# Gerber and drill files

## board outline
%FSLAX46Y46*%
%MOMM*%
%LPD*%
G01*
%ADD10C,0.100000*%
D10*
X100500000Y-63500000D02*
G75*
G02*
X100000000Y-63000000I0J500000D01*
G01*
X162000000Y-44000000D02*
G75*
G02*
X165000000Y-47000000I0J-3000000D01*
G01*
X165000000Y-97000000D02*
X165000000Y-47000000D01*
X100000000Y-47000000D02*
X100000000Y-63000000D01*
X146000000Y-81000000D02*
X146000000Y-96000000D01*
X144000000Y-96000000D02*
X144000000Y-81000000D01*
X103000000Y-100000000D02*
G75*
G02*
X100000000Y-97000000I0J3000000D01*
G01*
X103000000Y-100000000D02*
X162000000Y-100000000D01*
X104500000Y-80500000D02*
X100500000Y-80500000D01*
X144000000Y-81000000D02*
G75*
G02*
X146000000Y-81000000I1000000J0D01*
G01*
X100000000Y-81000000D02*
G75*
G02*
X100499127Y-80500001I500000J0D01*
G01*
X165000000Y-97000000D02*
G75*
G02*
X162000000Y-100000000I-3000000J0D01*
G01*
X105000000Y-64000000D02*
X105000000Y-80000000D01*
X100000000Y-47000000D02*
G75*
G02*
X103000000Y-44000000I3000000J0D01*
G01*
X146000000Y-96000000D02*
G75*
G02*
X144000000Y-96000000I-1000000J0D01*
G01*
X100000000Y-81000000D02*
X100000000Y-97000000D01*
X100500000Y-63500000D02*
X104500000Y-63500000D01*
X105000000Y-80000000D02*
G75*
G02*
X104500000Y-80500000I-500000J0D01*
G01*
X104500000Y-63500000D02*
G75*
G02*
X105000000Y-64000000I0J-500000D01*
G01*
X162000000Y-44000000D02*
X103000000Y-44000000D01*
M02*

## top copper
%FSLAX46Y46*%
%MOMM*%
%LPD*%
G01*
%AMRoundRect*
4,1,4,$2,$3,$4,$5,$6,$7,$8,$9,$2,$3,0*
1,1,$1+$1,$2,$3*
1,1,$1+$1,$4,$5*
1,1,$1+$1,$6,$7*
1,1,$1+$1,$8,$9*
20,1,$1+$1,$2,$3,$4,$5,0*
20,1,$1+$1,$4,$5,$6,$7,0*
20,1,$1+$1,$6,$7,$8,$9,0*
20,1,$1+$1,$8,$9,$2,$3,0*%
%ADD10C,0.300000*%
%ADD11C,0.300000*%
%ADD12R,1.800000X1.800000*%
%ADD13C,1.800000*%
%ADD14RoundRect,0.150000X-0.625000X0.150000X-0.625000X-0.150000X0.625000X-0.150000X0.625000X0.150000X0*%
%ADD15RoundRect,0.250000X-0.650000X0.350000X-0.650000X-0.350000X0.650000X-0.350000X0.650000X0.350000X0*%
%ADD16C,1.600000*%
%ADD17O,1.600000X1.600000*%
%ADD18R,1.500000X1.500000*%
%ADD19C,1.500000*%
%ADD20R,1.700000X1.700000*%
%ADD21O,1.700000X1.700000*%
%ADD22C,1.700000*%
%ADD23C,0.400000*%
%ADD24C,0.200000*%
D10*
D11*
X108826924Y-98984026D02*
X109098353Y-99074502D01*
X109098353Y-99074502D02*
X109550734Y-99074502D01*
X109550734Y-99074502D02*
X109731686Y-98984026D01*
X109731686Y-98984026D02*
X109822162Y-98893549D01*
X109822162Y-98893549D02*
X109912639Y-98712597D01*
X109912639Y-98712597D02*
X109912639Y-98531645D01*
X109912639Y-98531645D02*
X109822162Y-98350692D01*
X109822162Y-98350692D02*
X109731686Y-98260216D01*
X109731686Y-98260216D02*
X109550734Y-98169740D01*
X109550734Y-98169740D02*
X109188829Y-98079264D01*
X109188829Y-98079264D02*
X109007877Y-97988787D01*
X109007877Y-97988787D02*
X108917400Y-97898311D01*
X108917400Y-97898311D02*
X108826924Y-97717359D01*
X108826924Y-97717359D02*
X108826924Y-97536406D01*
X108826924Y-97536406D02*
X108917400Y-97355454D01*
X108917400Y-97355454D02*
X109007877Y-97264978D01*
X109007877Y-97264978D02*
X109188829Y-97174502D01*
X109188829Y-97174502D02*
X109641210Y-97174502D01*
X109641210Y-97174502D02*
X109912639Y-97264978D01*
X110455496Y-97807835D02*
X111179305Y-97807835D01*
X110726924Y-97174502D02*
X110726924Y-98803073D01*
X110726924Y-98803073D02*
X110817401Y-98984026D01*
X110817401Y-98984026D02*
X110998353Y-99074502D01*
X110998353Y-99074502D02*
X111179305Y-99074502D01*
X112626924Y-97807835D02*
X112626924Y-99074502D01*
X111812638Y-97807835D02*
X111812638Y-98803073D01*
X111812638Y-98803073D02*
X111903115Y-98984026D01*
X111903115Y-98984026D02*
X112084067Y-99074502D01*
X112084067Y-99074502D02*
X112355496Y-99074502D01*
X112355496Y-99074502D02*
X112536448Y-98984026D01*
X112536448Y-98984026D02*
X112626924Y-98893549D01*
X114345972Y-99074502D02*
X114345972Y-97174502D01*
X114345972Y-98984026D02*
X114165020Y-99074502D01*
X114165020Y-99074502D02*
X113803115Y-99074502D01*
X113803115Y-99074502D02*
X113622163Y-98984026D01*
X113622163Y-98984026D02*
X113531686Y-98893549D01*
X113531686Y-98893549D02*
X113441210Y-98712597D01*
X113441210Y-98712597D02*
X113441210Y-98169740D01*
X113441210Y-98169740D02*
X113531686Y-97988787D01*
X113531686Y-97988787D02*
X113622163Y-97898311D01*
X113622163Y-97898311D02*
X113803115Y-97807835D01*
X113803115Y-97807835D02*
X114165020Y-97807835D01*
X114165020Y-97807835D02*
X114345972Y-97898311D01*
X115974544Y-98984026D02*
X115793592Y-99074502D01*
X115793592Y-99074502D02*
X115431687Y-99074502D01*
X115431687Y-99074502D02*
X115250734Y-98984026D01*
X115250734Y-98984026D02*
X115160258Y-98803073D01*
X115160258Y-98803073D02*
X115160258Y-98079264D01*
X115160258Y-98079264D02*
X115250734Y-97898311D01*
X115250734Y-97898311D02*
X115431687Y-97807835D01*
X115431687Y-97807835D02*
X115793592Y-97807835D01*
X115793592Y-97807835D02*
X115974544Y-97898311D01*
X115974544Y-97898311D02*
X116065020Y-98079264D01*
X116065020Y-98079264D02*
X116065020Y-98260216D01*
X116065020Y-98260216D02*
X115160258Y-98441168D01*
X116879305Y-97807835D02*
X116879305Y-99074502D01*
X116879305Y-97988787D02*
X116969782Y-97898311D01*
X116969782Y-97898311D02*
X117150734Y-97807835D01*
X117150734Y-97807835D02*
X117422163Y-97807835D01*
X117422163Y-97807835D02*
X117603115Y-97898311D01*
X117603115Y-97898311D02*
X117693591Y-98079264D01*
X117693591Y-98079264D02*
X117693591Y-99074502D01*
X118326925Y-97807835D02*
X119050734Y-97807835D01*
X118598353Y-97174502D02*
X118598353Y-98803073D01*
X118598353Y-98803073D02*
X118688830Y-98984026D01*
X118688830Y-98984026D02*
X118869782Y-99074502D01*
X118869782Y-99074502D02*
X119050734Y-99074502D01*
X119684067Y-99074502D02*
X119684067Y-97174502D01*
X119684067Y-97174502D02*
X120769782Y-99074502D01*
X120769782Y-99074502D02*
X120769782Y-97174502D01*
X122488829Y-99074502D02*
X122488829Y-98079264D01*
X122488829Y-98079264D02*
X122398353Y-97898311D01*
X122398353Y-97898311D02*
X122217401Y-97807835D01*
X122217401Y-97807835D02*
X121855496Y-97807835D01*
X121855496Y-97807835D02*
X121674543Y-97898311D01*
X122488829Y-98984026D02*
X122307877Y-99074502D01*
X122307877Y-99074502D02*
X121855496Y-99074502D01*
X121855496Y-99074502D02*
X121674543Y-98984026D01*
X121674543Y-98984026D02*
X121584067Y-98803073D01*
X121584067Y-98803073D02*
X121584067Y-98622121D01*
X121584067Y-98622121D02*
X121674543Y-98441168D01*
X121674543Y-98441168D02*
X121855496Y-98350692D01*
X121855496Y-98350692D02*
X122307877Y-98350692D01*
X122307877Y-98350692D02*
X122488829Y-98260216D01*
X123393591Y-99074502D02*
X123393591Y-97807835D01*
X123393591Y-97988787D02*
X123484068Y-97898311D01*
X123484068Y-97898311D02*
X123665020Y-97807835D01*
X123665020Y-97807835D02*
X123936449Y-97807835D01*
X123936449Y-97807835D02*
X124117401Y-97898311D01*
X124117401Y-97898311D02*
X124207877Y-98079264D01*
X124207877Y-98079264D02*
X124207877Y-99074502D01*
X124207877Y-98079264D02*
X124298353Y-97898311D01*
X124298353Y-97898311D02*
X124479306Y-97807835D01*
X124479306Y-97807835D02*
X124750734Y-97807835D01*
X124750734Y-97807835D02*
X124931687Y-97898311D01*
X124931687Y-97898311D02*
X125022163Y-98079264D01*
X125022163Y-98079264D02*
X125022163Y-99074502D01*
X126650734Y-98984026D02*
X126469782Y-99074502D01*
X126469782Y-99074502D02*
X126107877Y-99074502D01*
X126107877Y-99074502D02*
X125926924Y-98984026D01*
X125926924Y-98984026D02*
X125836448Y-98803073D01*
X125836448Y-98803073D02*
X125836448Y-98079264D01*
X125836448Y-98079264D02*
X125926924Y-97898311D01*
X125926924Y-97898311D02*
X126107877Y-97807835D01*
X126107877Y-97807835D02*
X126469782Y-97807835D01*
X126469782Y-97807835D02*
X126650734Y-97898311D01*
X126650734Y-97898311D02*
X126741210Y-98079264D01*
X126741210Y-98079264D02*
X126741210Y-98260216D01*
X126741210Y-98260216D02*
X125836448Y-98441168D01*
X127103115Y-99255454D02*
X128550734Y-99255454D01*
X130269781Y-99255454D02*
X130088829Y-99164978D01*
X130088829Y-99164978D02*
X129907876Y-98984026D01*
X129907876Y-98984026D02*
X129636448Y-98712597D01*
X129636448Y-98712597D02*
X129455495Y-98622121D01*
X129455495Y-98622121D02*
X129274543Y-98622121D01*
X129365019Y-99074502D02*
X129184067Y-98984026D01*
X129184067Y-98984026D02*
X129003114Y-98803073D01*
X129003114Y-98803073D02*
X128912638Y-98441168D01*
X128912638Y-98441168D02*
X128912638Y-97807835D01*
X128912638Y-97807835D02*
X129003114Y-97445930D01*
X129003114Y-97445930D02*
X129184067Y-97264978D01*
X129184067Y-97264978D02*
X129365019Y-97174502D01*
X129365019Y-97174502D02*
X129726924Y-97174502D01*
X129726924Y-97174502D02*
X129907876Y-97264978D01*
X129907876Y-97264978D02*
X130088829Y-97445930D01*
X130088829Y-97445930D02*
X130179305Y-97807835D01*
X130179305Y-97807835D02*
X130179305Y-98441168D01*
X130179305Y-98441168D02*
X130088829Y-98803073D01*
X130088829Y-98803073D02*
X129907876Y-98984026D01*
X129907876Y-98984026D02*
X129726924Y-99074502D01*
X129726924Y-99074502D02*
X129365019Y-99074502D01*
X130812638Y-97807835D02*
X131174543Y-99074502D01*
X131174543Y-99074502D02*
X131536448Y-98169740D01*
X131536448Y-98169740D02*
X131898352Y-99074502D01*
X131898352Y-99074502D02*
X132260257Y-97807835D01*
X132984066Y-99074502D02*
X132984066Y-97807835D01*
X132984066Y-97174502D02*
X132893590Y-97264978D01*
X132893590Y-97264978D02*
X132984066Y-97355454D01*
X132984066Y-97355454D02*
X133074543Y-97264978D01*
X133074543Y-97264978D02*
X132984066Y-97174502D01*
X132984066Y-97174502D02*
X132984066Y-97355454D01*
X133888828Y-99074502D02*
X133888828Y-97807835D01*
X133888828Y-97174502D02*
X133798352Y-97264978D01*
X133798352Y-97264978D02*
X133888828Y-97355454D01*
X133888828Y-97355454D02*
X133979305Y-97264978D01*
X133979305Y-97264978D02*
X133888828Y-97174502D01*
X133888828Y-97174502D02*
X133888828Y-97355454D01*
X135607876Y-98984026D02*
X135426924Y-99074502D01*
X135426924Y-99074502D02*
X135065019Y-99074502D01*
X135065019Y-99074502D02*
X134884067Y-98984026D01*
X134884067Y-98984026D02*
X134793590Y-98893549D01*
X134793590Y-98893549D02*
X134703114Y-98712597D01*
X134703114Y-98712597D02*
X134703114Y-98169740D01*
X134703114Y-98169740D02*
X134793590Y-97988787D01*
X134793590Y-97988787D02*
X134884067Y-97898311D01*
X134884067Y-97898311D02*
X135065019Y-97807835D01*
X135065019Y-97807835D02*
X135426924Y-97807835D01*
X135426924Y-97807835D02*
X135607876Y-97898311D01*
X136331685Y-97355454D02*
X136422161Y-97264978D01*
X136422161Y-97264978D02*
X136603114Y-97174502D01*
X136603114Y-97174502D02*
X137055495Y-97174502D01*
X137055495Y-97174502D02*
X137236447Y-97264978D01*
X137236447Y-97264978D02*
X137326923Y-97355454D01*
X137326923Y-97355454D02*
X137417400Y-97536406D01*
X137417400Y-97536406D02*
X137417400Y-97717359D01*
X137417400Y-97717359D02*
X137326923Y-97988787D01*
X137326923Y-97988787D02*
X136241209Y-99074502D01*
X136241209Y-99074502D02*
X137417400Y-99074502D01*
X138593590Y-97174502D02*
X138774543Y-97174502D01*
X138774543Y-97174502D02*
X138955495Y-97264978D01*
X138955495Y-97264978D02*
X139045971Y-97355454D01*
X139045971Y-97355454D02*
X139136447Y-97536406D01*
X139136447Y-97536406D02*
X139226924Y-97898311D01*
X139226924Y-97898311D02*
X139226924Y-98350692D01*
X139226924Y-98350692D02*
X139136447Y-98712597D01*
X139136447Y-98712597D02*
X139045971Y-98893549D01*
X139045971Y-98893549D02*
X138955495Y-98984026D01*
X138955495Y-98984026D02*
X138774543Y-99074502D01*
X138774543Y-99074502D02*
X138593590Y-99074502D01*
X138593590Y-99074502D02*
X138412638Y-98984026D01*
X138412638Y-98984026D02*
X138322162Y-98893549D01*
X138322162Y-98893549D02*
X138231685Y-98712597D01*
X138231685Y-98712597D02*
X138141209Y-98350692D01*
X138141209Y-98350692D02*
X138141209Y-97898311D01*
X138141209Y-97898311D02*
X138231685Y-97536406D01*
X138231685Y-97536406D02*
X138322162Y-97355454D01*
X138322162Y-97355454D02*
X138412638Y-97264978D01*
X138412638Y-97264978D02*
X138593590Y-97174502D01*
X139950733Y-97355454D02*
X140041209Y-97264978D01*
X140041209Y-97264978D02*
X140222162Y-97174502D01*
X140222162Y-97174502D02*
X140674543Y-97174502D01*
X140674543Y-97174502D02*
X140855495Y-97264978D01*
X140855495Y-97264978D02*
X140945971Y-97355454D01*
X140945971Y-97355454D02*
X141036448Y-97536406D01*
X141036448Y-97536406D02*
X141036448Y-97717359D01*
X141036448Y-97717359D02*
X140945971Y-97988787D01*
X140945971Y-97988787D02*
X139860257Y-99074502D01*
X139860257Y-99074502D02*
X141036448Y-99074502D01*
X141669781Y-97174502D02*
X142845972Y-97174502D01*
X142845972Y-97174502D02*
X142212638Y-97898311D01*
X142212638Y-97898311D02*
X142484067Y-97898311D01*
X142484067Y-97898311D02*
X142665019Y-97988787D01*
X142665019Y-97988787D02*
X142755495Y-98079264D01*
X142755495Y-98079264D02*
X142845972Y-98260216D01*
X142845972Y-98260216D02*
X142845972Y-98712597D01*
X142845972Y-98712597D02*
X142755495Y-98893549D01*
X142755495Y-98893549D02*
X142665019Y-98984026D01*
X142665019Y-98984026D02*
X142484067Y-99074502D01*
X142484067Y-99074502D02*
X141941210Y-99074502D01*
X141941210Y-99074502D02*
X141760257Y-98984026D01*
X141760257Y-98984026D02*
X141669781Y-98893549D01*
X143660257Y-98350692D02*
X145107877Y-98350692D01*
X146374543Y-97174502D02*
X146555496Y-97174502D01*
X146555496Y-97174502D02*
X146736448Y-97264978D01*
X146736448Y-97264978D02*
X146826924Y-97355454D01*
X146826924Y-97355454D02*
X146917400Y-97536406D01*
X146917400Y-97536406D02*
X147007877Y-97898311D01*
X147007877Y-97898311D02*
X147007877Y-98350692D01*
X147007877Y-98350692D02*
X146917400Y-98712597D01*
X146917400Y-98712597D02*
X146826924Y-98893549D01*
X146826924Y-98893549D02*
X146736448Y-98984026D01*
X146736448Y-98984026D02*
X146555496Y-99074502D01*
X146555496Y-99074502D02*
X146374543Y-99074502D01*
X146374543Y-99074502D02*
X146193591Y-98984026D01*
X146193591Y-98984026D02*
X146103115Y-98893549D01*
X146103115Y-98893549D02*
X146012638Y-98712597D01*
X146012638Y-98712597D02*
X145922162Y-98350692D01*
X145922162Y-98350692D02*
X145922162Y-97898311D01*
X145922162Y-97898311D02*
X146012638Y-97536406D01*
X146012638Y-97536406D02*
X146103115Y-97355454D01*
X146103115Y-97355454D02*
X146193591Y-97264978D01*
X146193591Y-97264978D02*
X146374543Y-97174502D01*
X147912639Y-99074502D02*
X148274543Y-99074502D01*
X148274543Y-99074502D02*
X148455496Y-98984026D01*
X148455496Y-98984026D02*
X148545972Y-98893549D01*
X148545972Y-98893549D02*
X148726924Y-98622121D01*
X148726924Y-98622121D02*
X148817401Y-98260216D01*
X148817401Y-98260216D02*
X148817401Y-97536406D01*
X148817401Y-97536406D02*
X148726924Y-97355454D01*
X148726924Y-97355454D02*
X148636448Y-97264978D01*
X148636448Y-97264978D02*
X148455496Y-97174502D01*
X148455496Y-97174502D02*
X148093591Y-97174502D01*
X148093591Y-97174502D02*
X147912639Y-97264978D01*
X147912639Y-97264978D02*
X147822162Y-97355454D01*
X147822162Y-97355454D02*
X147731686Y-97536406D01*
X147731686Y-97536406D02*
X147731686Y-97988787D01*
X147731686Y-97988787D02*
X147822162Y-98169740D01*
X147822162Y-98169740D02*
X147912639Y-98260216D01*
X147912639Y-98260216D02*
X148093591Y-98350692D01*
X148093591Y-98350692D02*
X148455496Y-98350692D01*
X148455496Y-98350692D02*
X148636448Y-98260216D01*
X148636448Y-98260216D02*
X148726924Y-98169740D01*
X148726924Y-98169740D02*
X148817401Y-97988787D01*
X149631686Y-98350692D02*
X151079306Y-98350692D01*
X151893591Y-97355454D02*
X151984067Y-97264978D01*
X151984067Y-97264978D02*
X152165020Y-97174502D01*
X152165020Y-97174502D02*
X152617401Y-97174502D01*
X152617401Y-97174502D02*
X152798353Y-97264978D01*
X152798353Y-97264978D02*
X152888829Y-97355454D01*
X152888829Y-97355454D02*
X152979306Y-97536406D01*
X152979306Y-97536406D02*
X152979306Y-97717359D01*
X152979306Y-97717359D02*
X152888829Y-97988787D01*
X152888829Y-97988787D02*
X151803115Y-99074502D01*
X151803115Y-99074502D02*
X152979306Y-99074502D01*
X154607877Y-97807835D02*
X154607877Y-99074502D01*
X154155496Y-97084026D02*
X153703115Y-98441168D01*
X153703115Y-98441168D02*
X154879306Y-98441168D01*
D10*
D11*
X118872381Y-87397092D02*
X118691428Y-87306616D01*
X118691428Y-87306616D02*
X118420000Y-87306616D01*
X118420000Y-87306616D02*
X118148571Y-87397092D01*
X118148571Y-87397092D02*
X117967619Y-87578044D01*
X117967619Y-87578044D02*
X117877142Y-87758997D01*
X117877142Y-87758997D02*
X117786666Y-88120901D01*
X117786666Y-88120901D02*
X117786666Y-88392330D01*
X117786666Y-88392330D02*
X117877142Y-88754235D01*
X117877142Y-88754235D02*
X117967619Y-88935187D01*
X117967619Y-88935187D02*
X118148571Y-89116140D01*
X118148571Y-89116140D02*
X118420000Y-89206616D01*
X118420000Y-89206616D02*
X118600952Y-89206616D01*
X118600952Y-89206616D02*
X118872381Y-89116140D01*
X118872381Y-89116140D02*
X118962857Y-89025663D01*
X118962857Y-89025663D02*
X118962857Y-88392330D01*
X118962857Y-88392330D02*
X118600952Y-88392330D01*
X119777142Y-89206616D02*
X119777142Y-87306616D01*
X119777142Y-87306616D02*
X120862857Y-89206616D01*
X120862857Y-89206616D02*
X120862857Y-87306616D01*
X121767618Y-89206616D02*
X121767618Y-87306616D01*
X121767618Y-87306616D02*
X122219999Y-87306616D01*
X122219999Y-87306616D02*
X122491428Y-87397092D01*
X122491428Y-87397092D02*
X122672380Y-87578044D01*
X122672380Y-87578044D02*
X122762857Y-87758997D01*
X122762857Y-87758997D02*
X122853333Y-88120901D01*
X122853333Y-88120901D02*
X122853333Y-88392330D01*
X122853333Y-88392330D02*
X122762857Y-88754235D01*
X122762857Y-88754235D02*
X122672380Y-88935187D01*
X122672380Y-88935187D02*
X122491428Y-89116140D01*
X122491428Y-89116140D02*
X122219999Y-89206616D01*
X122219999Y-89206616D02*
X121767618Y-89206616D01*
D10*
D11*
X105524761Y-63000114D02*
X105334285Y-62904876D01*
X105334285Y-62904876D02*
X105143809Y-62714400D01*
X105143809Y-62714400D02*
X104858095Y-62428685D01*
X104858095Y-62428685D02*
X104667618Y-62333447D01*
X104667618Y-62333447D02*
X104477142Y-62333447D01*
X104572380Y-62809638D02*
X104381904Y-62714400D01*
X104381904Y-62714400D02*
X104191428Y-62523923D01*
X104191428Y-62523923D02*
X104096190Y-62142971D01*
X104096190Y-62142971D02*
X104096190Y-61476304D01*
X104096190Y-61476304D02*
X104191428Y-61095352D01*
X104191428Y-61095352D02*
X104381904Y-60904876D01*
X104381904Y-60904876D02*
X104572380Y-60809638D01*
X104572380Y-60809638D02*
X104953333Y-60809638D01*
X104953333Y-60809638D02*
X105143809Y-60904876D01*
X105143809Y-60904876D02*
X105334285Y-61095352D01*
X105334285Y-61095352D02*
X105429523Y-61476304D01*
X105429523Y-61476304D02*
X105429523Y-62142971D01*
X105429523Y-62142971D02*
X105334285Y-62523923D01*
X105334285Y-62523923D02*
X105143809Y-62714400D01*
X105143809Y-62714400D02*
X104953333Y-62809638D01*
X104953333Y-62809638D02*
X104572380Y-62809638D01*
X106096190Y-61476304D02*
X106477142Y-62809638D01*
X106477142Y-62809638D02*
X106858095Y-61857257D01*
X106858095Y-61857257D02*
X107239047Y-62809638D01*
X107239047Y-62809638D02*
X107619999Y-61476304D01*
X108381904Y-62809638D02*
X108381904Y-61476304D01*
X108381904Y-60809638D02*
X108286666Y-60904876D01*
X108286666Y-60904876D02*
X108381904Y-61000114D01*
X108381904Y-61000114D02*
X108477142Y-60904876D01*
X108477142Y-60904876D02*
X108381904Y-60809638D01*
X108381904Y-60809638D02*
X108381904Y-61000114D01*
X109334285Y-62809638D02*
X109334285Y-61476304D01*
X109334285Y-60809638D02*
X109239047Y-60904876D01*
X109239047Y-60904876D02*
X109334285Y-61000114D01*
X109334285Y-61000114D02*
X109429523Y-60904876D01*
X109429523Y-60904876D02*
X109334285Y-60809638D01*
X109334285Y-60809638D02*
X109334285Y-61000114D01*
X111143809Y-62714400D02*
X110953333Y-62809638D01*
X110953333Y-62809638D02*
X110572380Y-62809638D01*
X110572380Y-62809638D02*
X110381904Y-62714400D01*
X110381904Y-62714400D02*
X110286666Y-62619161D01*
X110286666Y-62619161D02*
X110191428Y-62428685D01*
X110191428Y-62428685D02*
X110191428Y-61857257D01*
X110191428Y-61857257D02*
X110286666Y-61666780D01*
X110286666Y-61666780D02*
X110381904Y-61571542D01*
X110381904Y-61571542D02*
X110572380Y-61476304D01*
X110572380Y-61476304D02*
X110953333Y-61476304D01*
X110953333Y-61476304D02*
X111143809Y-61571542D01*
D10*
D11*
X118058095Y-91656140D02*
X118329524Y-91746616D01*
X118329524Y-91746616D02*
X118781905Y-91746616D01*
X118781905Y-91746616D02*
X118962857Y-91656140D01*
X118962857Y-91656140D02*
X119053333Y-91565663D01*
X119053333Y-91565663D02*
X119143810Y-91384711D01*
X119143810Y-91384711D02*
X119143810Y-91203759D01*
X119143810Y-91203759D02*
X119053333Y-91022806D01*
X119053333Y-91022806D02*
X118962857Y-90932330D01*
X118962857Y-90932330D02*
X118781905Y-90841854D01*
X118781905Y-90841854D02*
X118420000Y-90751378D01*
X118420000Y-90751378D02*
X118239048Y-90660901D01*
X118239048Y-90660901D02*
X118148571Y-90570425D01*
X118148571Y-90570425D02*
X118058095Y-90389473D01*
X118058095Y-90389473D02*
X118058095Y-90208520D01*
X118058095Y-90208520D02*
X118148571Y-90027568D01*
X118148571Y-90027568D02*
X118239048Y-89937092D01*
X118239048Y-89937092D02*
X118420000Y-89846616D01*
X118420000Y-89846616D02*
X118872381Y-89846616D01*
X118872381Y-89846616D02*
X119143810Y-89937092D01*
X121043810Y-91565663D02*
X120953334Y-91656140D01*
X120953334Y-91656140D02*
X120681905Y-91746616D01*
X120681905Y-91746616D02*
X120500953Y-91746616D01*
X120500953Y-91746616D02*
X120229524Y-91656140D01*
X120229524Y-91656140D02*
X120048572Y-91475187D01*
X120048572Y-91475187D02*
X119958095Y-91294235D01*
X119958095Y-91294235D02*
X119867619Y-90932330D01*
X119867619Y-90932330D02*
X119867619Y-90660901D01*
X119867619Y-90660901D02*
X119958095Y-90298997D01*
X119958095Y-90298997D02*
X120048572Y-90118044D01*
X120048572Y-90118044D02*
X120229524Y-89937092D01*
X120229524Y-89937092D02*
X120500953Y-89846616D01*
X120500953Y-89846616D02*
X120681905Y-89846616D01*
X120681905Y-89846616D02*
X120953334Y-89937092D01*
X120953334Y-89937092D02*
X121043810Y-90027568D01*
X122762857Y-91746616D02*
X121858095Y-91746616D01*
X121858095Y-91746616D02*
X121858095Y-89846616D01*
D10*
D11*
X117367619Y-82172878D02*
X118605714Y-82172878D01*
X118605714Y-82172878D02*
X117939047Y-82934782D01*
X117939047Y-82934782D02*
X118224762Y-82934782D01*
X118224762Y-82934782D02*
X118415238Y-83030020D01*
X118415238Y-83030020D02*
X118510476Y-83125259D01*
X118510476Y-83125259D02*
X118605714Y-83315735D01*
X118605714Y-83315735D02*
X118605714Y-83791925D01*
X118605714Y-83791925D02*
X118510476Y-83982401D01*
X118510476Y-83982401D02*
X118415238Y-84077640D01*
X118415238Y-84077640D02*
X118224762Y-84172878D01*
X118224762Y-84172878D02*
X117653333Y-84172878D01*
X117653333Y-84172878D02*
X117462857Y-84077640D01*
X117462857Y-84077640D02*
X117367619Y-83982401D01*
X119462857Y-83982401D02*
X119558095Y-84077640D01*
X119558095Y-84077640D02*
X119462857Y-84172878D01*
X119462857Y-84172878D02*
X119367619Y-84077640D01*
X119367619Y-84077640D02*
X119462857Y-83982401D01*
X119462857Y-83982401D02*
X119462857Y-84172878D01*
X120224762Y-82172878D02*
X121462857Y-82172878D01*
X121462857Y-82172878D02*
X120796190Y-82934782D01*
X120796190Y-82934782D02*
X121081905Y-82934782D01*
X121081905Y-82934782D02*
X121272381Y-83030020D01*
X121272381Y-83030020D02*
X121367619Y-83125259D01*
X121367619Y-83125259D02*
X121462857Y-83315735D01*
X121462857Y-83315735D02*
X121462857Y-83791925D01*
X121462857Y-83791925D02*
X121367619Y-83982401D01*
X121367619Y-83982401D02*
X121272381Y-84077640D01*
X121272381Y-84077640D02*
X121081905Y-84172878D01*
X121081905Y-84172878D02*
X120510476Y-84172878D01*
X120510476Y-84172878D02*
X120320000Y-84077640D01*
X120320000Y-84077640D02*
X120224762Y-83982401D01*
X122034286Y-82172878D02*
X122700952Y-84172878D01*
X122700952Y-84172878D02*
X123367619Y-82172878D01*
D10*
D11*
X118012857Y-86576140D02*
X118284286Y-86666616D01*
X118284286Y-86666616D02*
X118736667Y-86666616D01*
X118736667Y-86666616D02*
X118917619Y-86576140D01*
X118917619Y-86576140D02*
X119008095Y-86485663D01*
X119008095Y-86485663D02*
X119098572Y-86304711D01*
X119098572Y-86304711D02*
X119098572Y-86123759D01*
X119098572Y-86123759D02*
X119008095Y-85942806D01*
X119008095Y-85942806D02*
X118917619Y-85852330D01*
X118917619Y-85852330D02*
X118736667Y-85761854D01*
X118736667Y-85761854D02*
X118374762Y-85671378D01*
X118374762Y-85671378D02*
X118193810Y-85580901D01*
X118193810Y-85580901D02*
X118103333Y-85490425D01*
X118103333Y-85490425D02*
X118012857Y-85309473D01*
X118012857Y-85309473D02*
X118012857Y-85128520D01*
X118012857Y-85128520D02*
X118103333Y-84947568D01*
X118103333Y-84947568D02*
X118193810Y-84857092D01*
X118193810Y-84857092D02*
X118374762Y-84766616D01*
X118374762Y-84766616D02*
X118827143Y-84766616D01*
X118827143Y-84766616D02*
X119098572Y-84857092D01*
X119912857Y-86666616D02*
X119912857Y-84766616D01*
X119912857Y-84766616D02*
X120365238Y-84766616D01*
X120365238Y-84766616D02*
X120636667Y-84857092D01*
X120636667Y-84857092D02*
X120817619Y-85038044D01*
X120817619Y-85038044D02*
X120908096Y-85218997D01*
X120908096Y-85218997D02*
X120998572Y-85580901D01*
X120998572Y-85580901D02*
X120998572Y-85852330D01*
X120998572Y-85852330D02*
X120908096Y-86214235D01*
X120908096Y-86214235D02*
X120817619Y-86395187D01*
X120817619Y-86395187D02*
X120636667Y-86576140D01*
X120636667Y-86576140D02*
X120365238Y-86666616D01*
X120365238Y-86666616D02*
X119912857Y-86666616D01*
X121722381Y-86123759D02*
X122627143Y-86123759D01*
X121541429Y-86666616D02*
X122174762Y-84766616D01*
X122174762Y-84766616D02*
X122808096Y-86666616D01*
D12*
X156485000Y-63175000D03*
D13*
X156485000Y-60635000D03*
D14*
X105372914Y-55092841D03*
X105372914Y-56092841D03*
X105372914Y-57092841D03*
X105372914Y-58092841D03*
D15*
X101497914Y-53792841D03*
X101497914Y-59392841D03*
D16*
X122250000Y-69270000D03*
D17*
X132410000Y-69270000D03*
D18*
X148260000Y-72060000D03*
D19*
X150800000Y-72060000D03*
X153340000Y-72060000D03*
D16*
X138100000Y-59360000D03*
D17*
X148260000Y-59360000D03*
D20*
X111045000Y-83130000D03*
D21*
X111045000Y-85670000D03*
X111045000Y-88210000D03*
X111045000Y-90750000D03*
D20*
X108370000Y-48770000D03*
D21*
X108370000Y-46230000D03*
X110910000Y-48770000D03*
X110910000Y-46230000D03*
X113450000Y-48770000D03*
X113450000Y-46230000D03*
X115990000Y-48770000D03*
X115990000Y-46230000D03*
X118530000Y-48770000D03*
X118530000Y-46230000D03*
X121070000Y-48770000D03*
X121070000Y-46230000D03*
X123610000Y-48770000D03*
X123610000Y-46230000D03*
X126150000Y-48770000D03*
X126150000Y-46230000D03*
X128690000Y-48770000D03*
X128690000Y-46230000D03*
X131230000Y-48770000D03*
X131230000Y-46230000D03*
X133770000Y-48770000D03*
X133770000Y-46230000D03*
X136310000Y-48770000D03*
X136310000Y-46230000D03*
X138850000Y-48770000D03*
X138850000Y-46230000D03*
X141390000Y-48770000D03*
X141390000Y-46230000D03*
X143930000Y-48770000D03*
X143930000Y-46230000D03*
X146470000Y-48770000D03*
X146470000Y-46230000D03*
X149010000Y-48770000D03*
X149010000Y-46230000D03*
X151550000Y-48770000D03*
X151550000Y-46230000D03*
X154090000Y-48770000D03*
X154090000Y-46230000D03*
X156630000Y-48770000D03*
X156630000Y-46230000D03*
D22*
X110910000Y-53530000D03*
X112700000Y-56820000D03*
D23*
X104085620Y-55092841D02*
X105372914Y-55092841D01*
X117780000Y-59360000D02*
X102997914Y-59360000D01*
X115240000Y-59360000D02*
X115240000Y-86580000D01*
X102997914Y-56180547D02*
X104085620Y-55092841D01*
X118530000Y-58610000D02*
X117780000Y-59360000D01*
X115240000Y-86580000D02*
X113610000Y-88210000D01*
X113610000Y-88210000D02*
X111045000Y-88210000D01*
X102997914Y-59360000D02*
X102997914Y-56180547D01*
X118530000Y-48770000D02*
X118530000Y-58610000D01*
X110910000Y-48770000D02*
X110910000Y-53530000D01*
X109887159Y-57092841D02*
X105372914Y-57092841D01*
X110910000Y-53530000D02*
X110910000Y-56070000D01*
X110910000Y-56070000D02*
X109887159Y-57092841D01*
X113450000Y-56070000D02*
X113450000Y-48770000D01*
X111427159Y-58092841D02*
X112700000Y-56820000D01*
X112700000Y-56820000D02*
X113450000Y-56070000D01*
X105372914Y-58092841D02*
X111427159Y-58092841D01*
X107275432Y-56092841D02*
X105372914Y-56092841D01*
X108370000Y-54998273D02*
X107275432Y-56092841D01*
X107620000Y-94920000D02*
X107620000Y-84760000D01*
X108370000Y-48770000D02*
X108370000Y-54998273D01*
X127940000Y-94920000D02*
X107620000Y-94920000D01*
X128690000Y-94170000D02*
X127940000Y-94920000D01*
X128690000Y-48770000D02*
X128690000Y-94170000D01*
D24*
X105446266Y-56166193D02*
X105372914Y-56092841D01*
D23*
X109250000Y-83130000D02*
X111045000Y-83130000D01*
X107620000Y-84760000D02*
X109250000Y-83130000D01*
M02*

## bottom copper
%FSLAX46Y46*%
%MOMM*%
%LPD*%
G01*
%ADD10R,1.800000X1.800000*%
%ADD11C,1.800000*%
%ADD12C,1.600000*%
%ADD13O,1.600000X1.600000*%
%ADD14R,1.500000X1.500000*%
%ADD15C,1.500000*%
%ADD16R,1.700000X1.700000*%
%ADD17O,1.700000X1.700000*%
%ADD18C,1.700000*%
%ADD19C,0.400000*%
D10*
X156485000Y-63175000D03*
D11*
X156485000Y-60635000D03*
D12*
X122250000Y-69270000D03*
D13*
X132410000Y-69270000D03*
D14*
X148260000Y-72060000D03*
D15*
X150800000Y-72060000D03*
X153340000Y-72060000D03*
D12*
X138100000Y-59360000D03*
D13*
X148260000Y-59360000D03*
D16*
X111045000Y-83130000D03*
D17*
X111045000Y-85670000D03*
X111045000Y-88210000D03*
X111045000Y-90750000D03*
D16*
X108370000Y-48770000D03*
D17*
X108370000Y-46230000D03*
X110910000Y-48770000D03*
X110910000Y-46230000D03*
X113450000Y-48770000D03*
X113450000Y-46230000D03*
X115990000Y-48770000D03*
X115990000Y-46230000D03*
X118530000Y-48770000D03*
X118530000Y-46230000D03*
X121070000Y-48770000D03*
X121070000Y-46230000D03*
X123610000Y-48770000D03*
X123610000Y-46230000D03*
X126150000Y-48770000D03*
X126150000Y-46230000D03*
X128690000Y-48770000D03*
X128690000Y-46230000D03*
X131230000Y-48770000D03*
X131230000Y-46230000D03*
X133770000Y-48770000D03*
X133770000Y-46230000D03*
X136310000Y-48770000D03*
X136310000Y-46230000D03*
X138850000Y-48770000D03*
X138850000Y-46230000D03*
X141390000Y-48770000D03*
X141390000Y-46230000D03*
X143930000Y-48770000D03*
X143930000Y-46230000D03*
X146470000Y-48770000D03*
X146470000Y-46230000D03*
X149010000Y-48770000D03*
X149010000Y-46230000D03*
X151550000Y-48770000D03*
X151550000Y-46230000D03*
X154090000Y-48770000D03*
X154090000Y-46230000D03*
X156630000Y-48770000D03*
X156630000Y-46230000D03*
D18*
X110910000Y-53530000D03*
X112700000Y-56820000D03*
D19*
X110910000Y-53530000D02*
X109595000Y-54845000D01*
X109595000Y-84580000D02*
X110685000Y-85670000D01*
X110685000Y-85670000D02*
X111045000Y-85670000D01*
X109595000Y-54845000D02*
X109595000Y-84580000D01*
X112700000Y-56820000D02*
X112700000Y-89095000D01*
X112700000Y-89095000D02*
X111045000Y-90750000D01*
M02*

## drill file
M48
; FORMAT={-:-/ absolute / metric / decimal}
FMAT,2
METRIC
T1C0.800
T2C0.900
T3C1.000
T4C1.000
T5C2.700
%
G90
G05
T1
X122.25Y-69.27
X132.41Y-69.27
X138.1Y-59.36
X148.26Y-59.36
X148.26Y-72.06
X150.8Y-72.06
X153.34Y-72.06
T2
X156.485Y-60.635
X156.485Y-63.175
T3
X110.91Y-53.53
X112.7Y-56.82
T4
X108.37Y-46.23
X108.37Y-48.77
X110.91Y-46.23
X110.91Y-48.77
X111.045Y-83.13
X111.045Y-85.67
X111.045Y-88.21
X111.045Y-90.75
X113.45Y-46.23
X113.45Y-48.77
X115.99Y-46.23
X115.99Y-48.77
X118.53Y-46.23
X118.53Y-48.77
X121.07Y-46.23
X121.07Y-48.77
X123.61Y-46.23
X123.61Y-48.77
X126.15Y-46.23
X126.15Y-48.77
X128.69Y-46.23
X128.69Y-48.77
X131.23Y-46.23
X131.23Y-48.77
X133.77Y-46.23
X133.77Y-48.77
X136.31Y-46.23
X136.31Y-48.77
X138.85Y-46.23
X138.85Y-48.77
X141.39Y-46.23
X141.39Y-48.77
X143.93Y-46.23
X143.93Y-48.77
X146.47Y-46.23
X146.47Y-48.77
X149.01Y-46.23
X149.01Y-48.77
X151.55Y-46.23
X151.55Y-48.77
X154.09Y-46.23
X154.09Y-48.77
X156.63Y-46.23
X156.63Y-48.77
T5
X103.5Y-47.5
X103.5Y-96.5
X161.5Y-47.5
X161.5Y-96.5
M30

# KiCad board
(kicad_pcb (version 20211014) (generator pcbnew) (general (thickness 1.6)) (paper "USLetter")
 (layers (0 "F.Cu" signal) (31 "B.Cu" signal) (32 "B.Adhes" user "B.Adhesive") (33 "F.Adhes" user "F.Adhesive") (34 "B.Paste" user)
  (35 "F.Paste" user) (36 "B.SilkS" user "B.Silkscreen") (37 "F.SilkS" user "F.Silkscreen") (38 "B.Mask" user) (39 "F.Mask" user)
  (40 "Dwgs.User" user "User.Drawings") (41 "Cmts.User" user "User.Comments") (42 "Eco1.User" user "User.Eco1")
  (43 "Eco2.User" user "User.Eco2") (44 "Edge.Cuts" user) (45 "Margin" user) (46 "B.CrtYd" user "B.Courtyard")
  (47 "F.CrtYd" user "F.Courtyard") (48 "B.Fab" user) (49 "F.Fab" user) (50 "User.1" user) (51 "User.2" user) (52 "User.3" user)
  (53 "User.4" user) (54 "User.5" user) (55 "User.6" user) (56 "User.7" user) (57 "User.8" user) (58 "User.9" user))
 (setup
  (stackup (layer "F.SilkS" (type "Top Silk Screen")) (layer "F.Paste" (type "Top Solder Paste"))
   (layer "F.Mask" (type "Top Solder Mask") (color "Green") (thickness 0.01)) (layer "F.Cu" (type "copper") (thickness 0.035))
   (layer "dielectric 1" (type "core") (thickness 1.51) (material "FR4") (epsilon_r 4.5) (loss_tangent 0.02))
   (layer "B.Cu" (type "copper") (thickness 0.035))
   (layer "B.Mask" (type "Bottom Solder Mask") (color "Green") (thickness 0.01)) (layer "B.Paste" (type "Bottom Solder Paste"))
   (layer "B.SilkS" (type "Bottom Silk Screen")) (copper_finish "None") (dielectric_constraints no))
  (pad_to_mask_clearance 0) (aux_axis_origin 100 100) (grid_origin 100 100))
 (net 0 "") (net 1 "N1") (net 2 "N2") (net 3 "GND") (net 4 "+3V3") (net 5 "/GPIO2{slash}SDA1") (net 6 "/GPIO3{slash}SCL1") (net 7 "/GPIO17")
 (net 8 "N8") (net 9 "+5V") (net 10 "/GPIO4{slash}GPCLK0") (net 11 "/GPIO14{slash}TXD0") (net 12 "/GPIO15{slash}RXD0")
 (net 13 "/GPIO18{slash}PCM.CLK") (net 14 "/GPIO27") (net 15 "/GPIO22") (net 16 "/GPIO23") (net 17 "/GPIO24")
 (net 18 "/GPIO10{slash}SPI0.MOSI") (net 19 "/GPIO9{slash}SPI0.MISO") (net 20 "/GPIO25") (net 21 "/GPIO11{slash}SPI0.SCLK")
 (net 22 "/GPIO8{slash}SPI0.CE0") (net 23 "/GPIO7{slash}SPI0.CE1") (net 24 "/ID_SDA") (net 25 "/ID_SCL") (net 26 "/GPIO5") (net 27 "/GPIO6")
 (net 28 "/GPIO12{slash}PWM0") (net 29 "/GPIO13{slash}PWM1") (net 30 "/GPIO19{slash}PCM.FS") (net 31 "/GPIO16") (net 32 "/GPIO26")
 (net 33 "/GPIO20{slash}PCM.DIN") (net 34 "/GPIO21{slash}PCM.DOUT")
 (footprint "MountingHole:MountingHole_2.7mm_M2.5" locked (layer "F.Cu") (at 161.5 47.5)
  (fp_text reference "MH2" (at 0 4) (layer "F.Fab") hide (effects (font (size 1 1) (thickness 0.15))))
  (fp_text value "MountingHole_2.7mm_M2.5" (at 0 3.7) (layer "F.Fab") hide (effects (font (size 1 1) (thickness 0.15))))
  (pad "" np_thru_hole circle locked (at 0 0) (size 2.7 2.7) (drill 2.7) (layers *.Cu *.Mask)))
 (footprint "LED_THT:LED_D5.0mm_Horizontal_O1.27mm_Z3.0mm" (layer "F.Cu") (at 156.485 63.175 90)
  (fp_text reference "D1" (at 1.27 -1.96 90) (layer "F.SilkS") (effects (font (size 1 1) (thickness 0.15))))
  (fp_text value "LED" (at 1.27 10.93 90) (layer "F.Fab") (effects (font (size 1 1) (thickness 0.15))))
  (pad "1" thru_hole rect (at 0 0 90) (size 1.8 1.8) (drill 0.9) (layers *.Cu *.Mask) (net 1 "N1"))
  (pad "2" thru_hole circle (at 2.54 0 90) (size 1.8 1.8) (drill 0.9) (layers *.Cu *.Mask) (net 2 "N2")))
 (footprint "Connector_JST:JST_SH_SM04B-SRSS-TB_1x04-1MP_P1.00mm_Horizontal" (layer "F.Cu") (at 103.372914 56.592841 -90)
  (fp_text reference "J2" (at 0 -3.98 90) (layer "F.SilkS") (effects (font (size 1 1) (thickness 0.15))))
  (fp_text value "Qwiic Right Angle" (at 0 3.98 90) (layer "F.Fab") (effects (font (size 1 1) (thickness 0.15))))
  (pad "1" smd roundrect (at -1.5 -2 270) (size 0.6 1.55) (layers "F.Cu" "F.Paste" "F.Mask") (roundrect_rratio 0.25) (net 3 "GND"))
  (pad "2" smd roundrect (at -0.5 -2 270) (size 0.6 1.55) (layers "F.Cu" "F.Paste" "F.Mask") (roundrect_rratio 0.25) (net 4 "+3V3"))
  (pad "3" smd roundrect (at 0.5 -2 270) (size 0.6 1.55) (layers "F.Cu" "F.Paste" "F.Mask") (roundrect_rratio 0.25)
   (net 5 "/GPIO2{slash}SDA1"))
  (pad "4" smd roundrect (at 1.5 -2 270) (size 0.6 1.55) (layers "F.Cu" "F.Paste" "F.Mask") (roundrect_rratio 0.25)
   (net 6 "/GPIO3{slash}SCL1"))
  (pad "MP" smd roundrect (at -2.8 1.875 270) (size 1.2 1.8) (layers "F.Cu" "F.Paste" "F.Mask") (roundrect_rratio 0.2083333333))
  (pad "MP" smd roundrect (at 2.8 1.875 270) (size 1.2 1.8) (layers "F.Cu" "F.Paste" "F.Mask") (roundrect_rratio 0.2083333333)))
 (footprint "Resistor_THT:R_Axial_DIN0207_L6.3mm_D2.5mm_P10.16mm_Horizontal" (layer "F.Cu") (at 122.25 69.27)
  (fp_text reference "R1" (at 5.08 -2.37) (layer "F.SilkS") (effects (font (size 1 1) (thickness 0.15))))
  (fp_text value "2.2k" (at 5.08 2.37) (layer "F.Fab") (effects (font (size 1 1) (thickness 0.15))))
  (pad "1" thru_hole circle (at 0 0) (size 1.6 1.6) (drill 0.8) (layers *.Cu *.Mask) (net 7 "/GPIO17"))
  (pad "2" thru_hole oval (at 10.16 0) (size 1.6 1.6) (drill 0.8) (layers *.Cu *.Mask) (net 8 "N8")))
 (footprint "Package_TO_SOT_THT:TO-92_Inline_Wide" (layer "F.Cu") (at 148.26 72.06)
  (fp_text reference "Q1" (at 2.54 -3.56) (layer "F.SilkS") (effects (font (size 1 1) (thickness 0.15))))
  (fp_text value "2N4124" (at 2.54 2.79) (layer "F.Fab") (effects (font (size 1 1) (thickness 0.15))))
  (pad "1" thru_hole rect (at 0 0) (size 1.5 1.5) (drill 0.8) (layers *.Cu *.Mask) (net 3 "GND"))
  (pad "2" thru_hole circle (at 2.54 0) (size 1.5 1.5) (drill 0.8) (layers *.Cu *.Mask) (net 8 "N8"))
  (pad "3" thru_hole circle (at 5.08 0) (size 1.5 1.5) (drill 0.8) (layers *.Cu *.Mask) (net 1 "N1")))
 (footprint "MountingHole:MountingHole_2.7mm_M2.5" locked (layer "F.Cu") (at 103.5 96.5)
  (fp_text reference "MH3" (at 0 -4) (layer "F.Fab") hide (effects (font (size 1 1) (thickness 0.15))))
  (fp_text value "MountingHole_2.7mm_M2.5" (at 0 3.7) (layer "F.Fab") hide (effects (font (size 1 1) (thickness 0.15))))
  (pad "" np_thru_hole circle locked (at 0 0) (size 2.7 2.7) (drill 2.7) (layers *.Cu *.Mask)))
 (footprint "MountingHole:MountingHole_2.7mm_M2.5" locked (layer "F.Cu") (at 103.5 47.5)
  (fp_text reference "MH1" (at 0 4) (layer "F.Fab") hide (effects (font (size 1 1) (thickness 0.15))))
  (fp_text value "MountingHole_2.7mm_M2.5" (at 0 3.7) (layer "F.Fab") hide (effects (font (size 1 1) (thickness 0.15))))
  (pad "" np_thru_hole circle locked (at 0 0) (size 2.7 2.7) (drill 2.7) (layers *.Cu *.Mask)))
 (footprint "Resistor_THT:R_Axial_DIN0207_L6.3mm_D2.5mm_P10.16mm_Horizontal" (layer "F.Cu") (at 138.1 59.36)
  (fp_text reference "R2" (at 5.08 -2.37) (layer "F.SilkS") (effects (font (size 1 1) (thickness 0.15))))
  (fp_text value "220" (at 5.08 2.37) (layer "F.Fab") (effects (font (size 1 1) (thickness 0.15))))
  (pad "1" thru_hole circle (at 0 0) (size 1.6 1.6) (drill 0.8) (layers *.Cu *.Mask) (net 4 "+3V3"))
  (pad "2" thru_hole oval (at 10.16 0) (size 1.6 1.6) (drill 0.8) (layers *.Cu *.Mask) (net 2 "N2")))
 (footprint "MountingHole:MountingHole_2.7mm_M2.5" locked (layer "F.Cu") (at 161.5 96.5)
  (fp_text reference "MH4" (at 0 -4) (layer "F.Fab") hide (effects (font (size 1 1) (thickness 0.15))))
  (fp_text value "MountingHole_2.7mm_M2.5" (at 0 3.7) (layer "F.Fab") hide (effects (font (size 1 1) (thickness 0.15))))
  (pad "" np_thru_hole circle locked (at 0 0) (size 2.7 2.7) (drill 2.7) (layers *.Cu *.Mask)))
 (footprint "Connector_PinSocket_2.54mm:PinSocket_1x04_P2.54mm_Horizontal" (layer "F.Cu") (at 111.045 83.13)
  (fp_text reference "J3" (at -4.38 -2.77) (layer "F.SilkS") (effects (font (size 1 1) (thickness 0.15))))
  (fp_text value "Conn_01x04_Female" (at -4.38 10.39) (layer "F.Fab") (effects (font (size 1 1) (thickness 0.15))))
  (pad "1" thru_hole rect (at 0 0) (size 1.7 1.7) (drill 1) (layers *.Cu *.Mask) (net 4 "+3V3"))
  (pad "2" thru_hole oval (at 0 2.54) (size 1.7 1.7) (drill 1) (layers *.Cu *.Mask) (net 5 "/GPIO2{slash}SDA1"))
  (pad "3" thru_hole oval (at 0 5.08) (size 1.7 1.7) (drill 1) (layers *.Cu *.Mask) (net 3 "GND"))
  (pad "4" thru_hole oval (at 0 7.62) (size 1.7 1.7) (drill 1) (layers *.Cu *.Mask) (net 6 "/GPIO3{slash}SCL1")))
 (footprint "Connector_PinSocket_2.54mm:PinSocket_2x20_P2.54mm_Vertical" (layer "B.Cu") (at 108.37 48.77 -90)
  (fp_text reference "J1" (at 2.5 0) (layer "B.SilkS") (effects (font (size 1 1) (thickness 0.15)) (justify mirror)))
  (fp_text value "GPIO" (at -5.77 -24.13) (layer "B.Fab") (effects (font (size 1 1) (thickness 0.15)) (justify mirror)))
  (pad "1" thru_hole rect locked (at 0 0 270) (size 1.7 1.7) (drill 1) (layers *.Cu *.Mask) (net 4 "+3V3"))
  (pad "2" thru_hole oval locked (at -2.54 0 270) (size 1.7 1.7) (drill 1) (layers *.Cu *.Mask) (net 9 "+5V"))
  (pad "3" thru_hole oval locked (at 0 -2.54 270) (size 1.7 1.7) (drill 1) (layers *.Cu *.Mask) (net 5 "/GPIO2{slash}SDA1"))
  (pad "4" thru_hole oval locked (at -2.54 -2.54 270) (size 1.7 1.7) (drill 1) (layers *.Cu *.Mask) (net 9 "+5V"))
  (pad "5" thru_hole oval locked (at 0 -5.08 270) (size 1.7 1.7) (drill 1) (layers *.Cu *.Mask) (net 6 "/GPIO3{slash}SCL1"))
  (pad "6" thru_hole oval locked (at -2.54 -5.08 270) (size 1.7 1.7) (drill 1) (layers *.Cu *.Mask) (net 3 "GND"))
  (pad "7" thru_hole oval locked (at 0 -7.62 270) (size 1.7 1.7) (drill 1) (layers *.Cu *.Mask) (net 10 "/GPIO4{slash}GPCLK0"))
  (pad "8" thru_hole oval locked (at -2.54 -7.62 270) (size 1.7 1.7) (drill 1) (layers *.Cu *.Mask) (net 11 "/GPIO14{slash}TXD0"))
  (pad "9" thru_hole oval locked (at 0 -10.16 270) (size 1.7 1.7) (drill 1) (layers *.Cu *.Mask) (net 3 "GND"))
  (pad "10" thru_hole oval locked (at -2.54 -10.16 270) (size 1.7 1.7) (drill 1) (layers *.Cu *.Mask) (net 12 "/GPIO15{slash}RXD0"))
  (pad "11" thru_hole oval locked (at 0 -12.7 270) (size 1.7 1.7) (drill 1) (layers *.Cu *.Mask) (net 7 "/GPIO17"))
  (pad "12" thru_hole oval locked (at -2.54 -12.7 270) (size 1.7 1.7) (drill 1) (layers *.Cu *.Mask) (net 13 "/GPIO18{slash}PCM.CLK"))
  (pad "13" thru_hole oval locked (at 0 -15.24 270) (size 1.7 1.7) (drill 1) (layers *.Cu *.Mask) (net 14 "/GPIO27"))
  (pad "14" thru_hole oval locked (at -2.54 -15.24 270) (size 1.7 1.7) (drill 1) (layers *.Cu *.Mask) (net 3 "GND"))
  (pad "15" thru_hole oval locked (at 0 -17.78 270) (size 1.7 1.7) (drill 1) (layers *.Cu *.Mask) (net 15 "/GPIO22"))
  (pad "16" thru_hole oval locked (at -2.54 -17.78 270) (size 1.7 1.7) (drill 1) (layers *.Cu *.Mask) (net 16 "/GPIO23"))
  (pad "17" thru_hole oval locked (at 0 -20.32 270) (size 1.7 1.7) (drill 1) (layers *.Cu *.Mask) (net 4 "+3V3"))
  (pad "18" thru_hole oval locked (at -2.54 -20.32 270) (size 1.7 1.7) (drill 1) (layers *.Cu *.Mask) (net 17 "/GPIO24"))
  (pad "19" thru_hole oval locked (at 0 -22.86 270) (size 1.7 1.7) (drill 1) (layers *.Cu *.Mask) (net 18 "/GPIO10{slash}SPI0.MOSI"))
  (pad "20" thru_hole oval locked (at -2.54 -22.86 270) (size 1.7 1.7) (drill 1) (layers *.Cu *.Mask) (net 3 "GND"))
  (pad "21" thru_hole oval locked (at 0 -25.4 270) (size 1.7 1.7) (drill 1) (layers *.Cu *.Mask) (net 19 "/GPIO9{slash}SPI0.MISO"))
  (pad "22" thru_hole oval locked (at -2.54 -25.4 270) (size 1.7 1.7) (drill 1) (layers *.Cu *.Mask) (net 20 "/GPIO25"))
  (pad "23" thru_hole oval locked (at 0 -27.94 270) (size 1.7 1.7) (drill 1) (layers *.Cu *.Mask) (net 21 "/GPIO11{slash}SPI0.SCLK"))
  (pad "24" thru_hole oval locked (at -2.54 -27.94 270) (size 1.7 1.7) (drill 1) (layers *.Cu *.Mask) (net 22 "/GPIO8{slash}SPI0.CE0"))
  (pad "25" thru_hole oval locked (at 0 -30.48 270) (size 1.7 1.7) (drill 1) (layers *.Cu *.Mask) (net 3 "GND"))
  (pad "26" thru_hole oval locked (at -2.54 -30.48 270) (size 1.7 1.7) (drill 1) (layers *.Cu *.Mask) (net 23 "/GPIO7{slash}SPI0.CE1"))
  (pad "27" thru_hole oval locked (at 0 -33.02 270) (size 1.7 1.7) (drill 1) (layers *.Cu *.Mask) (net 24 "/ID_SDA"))
  (pad "28" thru_hole oval locked (at -2.54 -33.02 270) (size 1.7 1.7) (drill 1) (layers *.Cu *.Mask) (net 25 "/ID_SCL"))
  (pad "29" thru_hole oval locked (at 0 -35.56 270) (size 1.7 1.7) (drill 1) (layers *.Cu *.Mask) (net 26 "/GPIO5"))
  (pad "30" thru_hole oval locked (at -2.54 -35.56 270) (size 1.7 1.7) (drill 1) (layers *.Cu *.Mask) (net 3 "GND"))
  (pad "31" thru_hole oval locked (at 0 -38.1 270) (size 1.7 1.7) (drill 1) (layers *.Cu *.Mask) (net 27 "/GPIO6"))
  (pad "32" thru_hole oval locked (at -2.54 -38.1 270) (size 1.7 1.7) (drill 1) (layers *.Cu *.Mask) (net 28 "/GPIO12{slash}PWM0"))
  (pad "33" thru_hole oval locked (at 0 -40.64 270) (size 1.7 1.7) (drill 1) (layers *.Cu *.Mask) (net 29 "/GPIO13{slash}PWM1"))
  (pad "34" thru_hole oval locked (at -2.54 -40.64 270) (size 1.7 1.7) (drill 1) (layers *.Cu *.Mask) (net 3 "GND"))
  (pad "35" thru_hole oval locked (at 0 -43.18 270) (size 1.7 1.7) (drill 1) (layers *.Cu *.Mask) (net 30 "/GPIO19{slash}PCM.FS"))
  (pad "36" thru_hole oval locked (at -2.54 -43.18 270) (size 1.7 1.7) (drill 1) (layers *.Cu *.Mask) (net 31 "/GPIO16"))
  (pad "37" thru_hole oval locked (at 0 -45.72 270) (size 1.7 1.7) (drill 1) (layers *.Cu *.Mask) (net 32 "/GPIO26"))
  (pad "38" thru_hole oval locked (at -2.54 -45.72 270) (size 1.7 1.7) (drill 1) (layers *.Cu *.Mask) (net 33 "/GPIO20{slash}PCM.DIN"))
  (pad "39" thru_hole oval locked (at 0 -48.26 270) (size 1.7 1.7) (drill 1) (layers *.Cu *.Mask) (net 3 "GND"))
  (pad "40" thru_hole oval locked (at -2.54 -48.26 270) (size 1.7 1.7) (drill 1) (layers *.Cu *.Mask) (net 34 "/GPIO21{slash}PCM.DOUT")))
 (gr_arc (start 100.5 63.5) (mid 100.146447 63.353553) (end 100 63) (layer "Edge.Cuts") (width 0.1))
 (gr_arc (start 162 44) (mid 164.12132 44.87868) (end 165 47) (layer "Edge.Cuts") (width 0.1))
 (gr_line (start 165 97) (end 165 47) (layer "Edge.Cuts") (width 0.1))
 (gr_line (start 100 47) (end 100 63) (layer "Edge.Cuts") (width 0.1))
 (gr_line (start 146 81) (end 146 96) (layer "Edge.Cuts") (width 0.1))
 (gr_line (start 144 96) (end 144 81) (layer "Edge.Cuts") (width 0.1))
 (gr_arc (start 103 100) (mid 100.87868 99.12132) (end 100 97) (layer "Edge.Cuts") (width 0.1))
 (gr_line (start 103 100) (end 162 100) (layer "Edge.Cuts") (width 0.1))
 (gr_line (start 104.5 80.5) (end 100.5 80.5) (layer "Edge.Cuts") (width 0.1))
 (gr_arc (start 144 81) (mid 145 80) (end 146 81) (layer "Edge.Cuts") (width 0.1))
 (gr_arc (start 100 81) (mid 100.146138 80.646755) (end 100.499127 80.500001) (layer "Edge.Cuts") (width 0.1))
 (gr_arc (start 165 97) (mid 164.12132 99.12132) (end 162 100) (layer "Edge.Cuts") (width 0.1))
 (gr_line (start 105 64) (end 105 80) (layer "Edge.Cuts") (width 0.1))
 (gr_arc (start 100 47) (mid 100.87868 44.87868) (end 103 44) (layer "Edge.Cuts") (width 0.1))
 (gr_arc (start 146 96) (mid 145 97) (end 144 96) (layer "Edge.Cuts") (width 0.1))
 (gr_line (start 100 81) (end 100 97) (layer "Edge.Cuts") (width 0.1))
 (gr_line (start 100.5 63.5) (end 104.5 63.5) (layer "Edge.Cuts") (width 0.1))
 (gr_arc (start 105 80) (mid 104.853553 80.353553) (end 104.5 80.5) (layer "Edge.Cuts") (width 0.1))
 (gr_arc (start 104.5 63.5) (mid 104.853553 63.646447) (end 105 64) (layer "Edge.Cuts") (width 0.1))
 (gr_line (start 162 44) (end 103 44) (layer "Edge.Cuts") (width 0.1))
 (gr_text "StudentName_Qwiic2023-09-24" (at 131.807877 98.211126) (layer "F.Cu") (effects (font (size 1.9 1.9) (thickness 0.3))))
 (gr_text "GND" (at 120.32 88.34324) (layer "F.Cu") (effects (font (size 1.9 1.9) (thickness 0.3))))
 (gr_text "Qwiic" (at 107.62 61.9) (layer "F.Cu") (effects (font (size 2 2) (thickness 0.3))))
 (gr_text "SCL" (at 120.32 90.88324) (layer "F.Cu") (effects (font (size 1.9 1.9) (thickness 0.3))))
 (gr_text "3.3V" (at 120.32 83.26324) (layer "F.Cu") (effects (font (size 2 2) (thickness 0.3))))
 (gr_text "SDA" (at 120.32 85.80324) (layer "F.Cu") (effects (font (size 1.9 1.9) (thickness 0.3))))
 (segment (start 104.08562 55.092841) (end 105.372914 55.092841) (width 0.4) (layer "F.Cu") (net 3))
 (segment (start 117.78 59.36) (end 102.997914 59.36) (width 0.4) (layer "F.Cu") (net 3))
 (segment (start 115.24 59.36) (end 115.24 86.58) (width 0.4) (layer "F.Cu") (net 3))
 (segment (start 102.997914 56.180547) (end 104.08562 55.092841) (width 0.4) (layer "F.Cu") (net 3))
 (segment (start 118.53 58.61) (end 117.78 59.36) (width 0.4) (layer "F.Cu") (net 3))
 (segment (start 115.24 86.58) (end 113.61 88.21) (width 0.4) (layer "F.Cu") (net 3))
 (segment (start 113.61 88.21) (end 111.045 88.21) (width 0.4) (layer "F.Cu") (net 3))
 (segment (start 102.997914 59.36) (end 102.997914 56.180547) (width 0.4) (layer "F.Cu") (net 3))
 (segment (start 118.53 48.77) (end 118.53 58.61) (width 0.4) (layer "F.Cu") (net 3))
 (segment (start 110.91 48.77) (end 110.91 53.53) (width 0.4) (layer "F.Cu") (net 5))
 (segment (start 109.887159 57.092841) (end 105.372914 57.092841) (width 0.4) (layer "F.Cu") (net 5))
 (segment (start 110.91 53.53) (end 110.91 56.07) (width 0.4) (layer "F.Cu") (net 5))
 (segment (start 110.91 56.07) (end 109.887159 57.092841) (width 0.4) (layer "F.Cu") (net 5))
 (via (at 110.91 53.53) (size 1.7) (drill 1) (layers "F.Cu" "B.Cu") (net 5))
 (segment (start 110.91 53.53) (end 109.595 54.845) (width 0.4) (layer "B.Cu") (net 5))
 (segment (start 109.595 84.58) (end 110.685 85.67) (width 0.4) (layer "B.Cu") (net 5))
 (segment (start 110.685 85.67) (end 111.045 85.67) (width 0.4) (layer "B.Cu") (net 5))
 (segment (start 109.595 54.845) (end 109.595 84.58) (width 0.4) (layer "B.Cu") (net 5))
 (segment (start 113.45 56.07) (end 113.45 48.77) (width 0.4) (layer "F.Cu") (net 6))
 (segment (start 111.427159 58.092841) (end 112.7 56.82) (width 0.4) (layer "F.Cu") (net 6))
 (segment (start 112.7 56.82) (end 113.45 56.07) (width 0.4) (layer "F.Cu") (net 6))
 (segment (start 105.372914 58.092841) (end 111.427159 58.092841) (width 0.4) (layer "F.Cu") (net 6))
 (via (at 112.7 56.82) (size 1.7) (drill 1) (layers "F.Cu" "B.Cu") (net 6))
 (segment (start 112.7 56.82) (end 112.7 89.095) (width 0.4) (layer "B.Cu") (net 6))
 (segment (start 112.7 89.095) (end 111.045 90.75) (width 0.4) (layer "B.Cu") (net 6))
 (segment (start 107.275432 56.092841) (end 105.372914 56.092841) (width 0.4) (layer "F.Cu") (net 4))
 (segment (start 108.37 54.998273) (end 107.275432 56.092841) (width 0.4) (layer "F.Cu") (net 4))
 (segment (start 107.62 94.92) (end 107.62 84.76) (width 0.4) (layer "F.Cu") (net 4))
 (segment (start 108.37 48.77) (end 108.37 54.998273) (width 0.4) (layer "F.Cu") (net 4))
 (segment (start 127.94 94.92) (end 107.62 94.92) (width 0.4) (layer "F.Cu") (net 4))
 (segment (start 128.69 94.17) (end 127.94 94.92) (width 0.4) (layer "F.Cu") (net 4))
 (segment (start 128.69 48.77) (end 128.69 94.17) (width 0.4) (layer "F.Cu") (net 4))
 (segment (start 105.446266 56.166193) (end 105.372914 56.092841) (width 0.2) (layer "F.Cu") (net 4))
 (segment (start 109.25 83.13) (end 111.045 83.13) (width 0.4) (layer "F.Cu") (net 4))
 (segment (start 107.62 84.76) (end 109.25 83.13) (width 0.4) (layer "F.Cu") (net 4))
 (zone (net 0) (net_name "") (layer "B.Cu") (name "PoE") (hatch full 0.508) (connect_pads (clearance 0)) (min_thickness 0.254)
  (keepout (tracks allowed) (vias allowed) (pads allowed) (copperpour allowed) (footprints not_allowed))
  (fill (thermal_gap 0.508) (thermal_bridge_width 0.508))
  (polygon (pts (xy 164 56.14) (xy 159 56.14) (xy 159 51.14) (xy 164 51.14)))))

